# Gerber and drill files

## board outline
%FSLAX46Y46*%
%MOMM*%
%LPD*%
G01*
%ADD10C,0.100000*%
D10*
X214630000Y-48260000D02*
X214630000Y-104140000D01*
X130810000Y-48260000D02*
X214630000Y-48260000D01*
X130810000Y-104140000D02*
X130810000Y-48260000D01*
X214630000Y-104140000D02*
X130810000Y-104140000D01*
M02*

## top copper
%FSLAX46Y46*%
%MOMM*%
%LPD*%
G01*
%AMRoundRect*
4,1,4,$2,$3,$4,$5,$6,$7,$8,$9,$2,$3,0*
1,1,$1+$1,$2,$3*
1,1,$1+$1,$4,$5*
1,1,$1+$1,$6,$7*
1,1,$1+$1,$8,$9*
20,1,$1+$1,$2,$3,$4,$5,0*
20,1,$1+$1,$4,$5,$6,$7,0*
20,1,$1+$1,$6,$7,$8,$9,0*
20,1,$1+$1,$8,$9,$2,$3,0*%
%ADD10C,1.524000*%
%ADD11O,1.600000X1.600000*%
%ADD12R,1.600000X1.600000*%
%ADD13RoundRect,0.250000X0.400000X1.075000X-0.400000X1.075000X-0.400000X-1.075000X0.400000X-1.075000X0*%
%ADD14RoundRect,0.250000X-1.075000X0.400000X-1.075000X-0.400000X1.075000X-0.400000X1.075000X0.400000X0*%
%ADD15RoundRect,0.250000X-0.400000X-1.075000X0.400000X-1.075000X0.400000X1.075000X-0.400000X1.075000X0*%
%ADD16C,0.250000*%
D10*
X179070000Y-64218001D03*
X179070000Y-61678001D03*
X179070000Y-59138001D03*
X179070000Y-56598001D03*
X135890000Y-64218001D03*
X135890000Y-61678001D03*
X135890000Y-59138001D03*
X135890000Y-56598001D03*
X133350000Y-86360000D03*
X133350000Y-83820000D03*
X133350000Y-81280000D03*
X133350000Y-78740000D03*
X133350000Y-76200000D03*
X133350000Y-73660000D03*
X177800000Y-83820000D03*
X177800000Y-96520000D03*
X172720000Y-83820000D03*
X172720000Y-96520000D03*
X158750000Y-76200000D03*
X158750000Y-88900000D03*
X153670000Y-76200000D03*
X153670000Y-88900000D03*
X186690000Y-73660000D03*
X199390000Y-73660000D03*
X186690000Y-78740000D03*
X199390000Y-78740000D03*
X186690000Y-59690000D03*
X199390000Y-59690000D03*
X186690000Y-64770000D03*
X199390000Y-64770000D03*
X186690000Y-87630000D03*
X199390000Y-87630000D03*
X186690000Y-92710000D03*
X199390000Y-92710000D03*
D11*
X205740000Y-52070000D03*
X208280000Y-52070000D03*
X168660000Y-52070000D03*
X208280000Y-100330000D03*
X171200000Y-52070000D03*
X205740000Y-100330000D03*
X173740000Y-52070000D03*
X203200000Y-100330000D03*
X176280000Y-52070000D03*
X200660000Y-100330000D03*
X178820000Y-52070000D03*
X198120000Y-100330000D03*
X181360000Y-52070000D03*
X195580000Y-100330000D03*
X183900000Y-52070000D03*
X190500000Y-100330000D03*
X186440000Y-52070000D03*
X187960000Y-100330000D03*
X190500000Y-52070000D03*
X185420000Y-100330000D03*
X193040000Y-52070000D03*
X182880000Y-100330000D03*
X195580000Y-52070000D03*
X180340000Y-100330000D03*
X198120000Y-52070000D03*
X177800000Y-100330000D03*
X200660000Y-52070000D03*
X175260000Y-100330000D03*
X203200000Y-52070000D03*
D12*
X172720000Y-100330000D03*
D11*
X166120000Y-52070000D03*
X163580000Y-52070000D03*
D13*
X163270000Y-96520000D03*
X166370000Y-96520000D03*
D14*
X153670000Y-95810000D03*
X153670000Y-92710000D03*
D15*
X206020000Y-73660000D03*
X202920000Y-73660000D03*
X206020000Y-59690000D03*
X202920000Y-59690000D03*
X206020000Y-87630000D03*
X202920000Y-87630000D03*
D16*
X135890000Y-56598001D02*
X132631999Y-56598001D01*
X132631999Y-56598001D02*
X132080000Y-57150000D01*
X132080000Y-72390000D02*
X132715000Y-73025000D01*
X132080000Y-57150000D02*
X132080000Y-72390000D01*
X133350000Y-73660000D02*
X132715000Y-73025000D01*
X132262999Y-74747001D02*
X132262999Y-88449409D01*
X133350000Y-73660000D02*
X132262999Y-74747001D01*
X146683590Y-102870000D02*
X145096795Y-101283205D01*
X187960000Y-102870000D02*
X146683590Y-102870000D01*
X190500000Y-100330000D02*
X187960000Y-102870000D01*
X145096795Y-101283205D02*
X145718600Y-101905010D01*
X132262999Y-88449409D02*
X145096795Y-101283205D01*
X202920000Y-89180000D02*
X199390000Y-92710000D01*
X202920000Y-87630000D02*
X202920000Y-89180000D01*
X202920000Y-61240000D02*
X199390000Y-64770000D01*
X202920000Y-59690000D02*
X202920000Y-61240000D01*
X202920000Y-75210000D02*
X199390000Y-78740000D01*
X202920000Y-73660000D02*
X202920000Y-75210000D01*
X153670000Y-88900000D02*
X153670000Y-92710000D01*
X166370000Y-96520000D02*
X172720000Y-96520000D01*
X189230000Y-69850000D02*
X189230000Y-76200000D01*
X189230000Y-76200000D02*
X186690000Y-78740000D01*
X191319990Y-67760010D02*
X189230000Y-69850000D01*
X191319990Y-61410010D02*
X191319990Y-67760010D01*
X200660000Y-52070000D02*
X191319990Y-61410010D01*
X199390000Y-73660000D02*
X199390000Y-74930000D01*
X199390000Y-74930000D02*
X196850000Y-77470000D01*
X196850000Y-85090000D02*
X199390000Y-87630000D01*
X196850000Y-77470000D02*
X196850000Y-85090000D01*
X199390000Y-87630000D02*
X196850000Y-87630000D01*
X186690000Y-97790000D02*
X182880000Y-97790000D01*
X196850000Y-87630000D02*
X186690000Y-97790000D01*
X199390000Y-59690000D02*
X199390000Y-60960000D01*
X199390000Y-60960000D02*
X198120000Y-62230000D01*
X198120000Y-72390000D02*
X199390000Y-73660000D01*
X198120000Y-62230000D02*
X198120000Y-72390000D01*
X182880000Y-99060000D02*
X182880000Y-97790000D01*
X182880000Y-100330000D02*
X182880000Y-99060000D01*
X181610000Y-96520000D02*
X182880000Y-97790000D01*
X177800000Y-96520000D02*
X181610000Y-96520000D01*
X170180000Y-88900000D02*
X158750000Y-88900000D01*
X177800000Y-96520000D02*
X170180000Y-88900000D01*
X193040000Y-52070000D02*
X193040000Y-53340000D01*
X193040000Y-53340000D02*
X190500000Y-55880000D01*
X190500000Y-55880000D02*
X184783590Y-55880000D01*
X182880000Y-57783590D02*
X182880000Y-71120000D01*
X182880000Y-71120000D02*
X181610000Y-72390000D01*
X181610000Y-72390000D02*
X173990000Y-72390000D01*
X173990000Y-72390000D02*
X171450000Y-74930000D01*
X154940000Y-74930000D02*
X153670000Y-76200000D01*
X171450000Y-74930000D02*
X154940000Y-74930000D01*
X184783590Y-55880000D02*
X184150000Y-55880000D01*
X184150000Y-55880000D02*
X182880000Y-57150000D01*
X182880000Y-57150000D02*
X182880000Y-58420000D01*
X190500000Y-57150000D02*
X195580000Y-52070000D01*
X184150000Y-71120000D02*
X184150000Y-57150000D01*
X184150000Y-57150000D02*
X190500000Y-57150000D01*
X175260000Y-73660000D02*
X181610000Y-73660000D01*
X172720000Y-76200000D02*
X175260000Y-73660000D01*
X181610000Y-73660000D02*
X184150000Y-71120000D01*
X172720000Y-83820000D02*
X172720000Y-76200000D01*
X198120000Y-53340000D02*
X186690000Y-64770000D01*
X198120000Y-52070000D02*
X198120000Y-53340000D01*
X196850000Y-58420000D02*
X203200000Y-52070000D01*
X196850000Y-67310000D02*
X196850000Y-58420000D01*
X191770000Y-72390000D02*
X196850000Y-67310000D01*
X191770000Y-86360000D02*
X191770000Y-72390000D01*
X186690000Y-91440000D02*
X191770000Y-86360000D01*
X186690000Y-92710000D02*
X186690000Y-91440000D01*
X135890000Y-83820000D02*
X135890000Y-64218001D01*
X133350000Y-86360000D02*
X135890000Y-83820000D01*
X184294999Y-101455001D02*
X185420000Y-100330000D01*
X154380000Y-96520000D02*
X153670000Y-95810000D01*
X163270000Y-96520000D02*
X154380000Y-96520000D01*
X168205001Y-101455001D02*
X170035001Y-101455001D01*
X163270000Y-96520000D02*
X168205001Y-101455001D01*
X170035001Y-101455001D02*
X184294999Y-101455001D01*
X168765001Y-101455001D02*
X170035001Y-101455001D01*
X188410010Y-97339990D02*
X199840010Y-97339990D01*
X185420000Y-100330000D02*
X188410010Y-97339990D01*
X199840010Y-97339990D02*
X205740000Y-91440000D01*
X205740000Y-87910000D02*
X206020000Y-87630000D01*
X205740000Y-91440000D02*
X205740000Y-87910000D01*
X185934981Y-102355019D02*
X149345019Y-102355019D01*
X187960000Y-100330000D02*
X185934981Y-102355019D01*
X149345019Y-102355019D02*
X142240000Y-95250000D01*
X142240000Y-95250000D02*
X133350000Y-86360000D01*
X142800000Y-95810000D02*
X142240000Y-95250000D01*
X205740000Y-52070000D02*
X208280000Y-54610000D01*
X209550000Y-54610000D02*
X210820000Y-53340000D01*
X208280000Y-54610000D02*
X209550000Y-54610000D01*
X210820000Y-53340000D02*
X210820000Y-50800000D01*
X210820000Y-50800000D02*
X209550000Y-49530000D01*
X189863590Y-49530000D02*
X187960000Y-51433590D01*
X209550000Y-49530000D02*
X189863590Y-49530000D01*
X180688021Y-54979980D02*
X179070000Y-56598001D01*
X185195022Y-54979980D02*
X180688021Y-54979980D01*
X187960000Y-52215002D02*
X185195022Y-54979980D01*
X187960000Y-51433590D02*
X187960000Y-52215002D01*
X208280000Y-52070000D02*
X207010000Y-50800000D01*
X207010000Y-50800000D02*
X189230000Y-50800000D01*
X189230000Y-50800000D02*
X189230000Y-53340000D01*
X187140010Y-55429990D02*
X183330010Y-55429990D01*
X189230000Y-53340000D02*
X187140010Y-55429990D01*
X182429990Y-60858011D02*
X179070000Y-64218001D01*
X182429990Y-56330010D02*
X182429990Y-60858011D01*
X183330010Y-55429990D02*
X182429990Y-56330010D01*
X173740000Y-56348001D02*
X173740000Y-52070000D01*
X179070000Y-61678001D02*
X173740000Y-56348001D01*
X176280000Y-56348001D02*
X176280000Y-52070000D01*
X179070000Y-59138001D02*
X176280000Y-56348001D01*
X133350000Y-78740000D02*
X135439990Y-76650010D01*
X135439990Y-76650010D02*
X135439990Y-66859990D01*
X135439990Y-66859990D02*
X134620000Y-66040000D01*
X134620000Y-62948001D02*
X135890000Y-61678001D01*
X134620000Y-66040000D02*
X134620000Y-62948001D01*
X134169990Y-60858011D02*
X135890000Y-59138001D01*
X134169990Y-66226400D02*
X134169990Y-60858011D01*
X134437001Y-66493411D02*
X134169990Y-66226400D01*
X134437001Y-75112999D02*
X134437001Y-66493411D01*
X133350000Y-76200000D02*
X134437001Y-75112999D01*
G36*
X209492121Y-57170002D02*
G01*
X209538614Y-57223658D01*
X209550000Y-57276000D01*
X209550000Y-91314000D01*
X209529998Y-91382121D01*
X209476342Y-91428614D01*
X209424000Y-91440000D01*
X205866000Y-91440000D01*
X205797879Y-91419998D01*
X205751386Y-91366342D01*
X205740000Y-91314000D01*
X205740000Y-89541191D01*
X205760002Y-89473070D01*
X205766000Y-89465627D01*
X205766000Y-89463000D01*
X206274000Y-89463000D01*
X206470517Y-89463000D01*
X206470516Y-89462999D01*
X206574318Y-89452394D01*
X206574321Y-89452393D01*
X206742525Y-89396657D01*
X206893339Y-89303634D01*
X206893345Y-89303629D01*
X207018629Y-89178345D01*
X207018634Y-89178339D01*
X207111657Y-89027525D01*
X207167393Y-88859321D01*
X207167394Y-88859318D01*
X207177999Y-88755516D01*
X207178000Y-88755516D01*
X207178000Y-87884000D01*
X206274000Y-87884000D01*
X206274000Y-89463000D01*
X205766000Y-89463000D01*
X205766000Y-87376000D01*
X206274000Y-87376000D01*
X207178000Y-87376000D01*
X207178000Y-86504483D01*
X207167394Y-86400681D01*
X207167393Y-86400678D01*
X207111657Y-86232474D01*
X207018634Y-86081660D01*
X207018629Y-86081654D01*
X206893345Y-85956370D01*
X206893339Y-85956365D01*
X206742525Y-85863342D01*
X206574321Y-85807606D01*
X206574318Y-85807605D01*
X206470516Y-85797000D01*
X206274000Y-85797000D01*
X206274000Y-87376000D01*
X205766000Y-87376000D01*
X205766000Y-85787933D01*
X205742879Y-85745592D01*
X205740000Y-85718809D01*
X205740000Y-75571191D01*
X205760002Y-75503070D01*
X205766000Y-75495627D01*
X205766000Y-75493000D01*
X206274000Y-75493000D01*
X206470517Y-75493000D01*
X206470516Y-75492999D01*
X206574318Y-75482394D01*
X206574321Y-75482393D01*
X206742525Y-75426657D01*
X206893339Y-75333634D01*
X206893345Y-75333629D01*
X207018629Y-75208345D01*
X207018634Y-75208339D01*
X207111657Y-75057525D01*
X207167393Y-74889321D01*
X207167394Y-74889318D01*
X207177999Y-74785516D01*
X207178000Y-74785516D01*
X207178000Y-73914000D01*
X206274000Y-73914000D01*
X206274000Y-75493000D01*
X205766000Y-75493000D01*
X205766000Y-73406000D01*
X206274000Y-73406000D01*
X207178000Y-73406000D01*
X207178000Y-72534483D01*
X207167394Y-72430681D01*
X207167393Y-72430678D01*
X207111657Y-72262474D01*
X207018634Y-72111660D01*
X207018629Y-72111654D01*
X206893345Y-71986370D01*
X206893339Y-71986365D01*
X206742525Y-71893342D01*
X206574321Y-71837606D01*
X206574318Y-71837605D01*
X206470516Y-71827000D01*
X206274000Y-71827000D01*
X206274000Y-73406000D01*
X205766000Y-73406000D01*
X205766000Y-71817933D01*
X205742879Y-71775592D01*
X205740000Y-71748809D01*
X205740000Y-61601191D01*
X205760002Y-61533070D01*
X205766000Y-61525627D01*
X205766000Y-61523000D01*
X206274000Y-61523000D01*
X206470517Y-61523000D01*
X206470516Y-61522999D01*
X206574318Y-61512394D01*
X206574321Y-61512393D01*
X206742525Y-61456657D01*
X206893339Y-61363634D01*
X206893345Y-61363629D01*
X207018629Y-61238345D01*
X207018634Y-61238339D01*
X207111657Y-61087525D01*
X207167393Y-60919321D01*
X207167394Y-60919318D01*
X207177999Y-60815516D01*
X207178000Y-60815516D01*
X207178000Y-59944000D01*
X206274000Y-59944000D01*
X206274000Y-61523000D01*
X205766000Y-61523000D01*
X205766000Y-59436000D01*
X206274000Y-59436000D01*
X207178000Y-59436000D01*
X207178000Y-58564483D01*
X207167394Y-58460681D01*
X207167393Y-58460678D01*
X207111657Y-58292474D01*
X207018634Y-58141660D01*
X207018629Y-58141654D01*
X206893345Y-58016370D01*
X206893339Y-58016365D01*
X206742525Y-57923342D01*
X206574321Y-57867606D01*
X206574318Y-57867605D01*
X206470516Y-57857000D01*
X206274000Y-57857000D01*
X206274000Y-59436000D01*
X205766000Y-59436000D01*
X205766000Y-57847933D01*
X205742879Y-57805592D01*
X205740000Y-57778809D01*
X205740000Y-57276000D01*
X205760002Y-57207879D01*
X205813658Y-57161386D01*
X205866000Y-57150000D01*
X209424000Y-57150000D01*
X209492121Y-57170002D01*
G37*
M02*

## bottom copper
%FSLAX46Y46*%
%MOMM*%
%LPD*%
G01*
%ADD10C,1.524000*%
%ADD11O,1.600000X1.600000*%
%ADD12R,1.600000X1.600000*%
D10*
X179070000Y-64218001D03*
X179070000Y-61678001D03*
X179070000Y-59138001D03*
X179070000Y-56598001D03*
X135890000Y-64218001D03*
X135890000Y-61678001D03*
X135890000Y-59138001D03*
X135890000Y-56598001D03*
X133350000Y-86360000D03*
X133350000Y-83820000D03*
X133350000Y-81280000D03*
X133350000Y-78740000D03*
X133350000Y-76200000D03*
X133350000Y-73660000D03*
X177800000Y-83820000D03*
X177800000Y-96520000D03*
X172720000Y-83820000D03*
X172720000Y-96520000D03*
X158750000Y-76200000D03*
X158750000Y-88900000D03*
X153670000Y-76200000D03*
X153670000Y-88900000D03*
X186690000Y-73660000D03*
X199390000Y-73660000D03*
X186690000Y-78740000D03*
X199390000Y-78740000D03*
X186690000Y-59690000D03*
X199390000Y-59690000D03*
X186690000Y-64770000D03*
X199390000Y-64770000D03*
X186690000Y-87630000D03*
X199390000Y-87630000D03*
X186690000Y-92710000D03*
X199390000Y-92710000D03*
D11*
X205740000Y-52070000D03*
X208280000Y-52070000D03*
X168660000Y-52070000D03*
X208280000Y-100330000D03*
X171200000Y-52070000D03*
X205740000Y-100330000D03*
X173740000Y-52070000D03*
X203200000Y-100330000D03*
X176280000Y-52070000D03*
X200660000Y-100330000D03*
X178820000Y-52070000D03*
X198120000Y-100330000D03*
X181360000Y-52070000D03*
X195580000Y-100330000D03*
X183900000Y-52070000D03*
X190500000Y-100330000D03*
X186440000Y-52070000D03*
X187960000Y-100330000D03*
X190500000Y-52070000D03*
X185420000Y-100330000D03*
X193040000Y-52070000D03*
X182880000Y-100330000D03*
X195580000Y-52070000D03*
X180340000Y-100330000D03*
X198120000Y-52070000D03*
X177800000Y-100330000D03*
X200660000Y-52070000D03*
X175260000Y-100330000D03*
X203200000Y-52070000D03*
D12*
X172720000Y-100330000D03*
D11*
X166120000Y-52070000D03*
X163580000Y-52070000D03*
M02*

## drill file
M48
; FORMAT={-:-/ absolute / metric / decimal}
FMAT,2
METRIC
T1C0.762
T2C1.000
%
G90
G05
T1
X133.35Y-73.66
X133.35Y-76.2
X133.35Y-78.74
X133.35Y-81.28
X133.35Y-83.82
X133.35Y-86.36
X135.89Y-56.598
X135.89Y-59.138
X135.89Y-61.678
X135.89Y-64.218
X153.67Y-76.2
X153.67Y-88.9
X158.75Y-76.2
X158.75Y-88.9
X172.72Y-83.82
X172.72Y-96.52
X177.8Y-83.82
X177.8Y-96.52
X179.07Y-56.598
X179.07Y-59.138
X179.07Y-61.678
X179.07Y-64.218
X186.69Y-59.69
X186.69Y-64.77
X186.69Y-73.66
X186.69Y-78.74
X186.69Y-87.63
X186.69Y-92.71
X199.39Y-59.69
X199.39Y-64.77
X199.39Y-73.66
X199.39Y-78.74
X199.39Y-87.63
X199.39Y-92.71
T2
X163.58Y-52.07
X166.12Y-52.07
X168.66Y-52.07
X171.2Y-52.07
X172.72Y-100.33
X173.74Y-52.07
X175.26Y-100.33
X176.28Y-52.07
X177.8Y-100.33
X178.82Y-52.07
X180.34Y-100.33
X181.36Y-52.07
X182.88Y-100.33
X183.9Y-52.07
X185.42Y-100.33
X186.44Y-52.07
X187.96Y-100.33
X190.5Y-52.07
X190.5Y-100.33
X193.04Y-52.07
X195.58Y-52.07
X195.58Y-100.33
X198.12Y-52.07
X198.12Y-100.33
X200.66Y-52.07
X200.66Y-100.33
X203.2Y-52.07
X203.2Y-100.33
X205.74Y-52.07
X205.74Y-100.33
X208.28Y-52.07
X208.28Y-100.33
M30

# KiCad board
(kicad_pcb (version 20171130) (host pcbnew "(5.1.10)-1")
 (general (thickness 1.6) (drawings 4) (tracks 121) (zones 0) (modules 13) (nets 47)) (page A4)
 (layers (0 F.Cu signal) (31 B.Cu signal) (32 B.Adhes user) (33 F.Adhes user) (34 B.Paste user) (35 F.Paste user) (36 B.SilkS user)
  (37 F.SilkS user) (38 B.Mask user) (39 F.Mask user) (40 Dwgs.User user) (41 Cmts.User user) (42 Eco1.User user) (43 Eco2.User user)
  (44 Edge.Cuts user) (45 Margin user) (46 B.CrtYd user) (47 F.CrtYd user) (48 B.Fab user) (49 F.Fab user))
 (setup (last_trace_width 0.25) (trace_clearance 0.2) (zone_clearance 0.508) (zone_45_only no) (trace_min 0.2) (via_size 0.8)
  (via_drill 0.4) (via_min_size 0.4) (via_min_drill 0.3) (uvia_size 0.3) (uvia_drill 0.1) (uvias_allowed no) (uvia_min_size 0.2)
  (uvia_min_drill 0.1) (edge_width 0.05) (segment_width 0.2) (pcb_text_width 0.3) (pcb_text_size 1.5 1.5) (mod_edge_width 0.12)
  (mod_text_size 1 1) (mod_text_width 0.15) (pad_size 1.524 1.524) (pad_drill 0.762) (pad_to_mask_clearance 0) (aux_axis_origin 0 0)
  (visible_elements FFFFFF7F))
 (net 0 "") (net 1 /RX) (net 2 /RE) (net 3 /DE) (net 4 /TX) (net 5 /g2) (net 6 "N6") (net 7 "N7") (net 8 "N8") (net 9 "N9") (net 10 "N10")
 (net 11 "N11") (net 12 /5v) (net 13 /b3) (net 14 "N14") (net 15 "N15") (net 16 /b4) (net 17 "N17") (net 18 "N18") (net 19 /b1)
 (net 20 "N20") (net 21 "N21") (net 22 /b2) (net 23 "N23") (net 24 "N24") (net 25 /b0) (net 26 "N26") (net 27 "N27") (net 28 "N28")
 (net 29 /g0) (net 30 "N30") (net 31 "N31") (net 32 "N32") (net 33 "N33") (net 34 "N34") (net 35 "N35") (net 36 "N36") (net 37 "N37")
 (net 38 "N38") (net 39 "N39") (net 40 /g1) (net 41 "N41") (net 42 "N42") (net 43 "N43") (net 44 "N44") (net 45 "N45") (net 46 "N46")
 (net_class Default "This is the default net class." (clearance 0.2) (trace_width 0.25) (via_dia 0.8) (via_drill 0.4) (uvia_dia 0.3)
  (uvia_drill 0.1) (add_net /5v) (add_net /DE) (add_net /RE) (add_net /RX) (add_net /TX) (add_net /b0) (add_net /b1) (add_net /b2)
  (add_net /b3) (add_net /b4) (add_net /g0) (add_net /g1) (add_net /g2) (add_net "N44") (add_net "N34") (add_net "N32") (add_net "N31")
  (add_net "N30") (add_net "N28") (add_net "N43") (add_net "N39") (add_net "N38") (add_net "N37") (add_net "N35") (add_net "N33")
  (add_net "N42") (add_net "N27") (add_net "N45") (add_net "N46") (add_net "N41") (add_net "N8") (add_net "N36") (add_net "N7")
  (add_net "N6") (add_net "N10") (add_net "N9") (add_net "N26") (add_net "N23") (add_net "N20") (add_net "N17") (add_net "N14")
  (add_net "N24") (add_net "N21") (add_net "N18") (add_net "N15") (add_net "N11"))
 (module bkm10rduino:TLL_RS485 (layer F.Cu) (at 157.48 61.678001)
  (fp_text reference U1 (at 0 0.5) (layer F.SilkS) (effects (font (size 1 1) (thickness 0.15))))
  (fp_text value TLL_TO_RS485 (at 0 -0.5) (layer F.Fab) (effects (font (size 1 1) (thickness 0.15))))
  (pad 8 thru_hole circle (at 21.59 2.54) (size 1.524 1.524) (drill 0.762) (layers *.Cu *.Mask) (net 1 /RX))
  (pad 7 thru_hole circle (at 21.59 0) (size 1.524 1.524) (drill 0.762) (layers *.Cu *.Mask) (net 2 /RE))
  (pad 6 thru_hole circle (at 21.59 -2.54) (size 1.524 1.524) (drill 0.762) (layers *.Cu *.Mask) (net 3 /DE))
  (pad 5 thru_hole circle (at 21.59 -5.08) (size 1.524 1.524) (drill 0.762) (layers *.Cu *.Mask) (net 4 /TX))
  (pad 4 thru_hole circle (at -21.59 2.54) (size 1.524 1.524) (drill 0.762) (layers *.Cu *.Mask) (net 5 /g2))
  (pad 3 thru_hole circle (at -21.59 0) (size 1.524 1.524) (drill 0.762) (layers *.Cu *.Mask) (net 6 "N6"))
  (pad 2 thru_hole circle (at -21.59 -2.54) (size 1.524 1.524) (drill 0.762) (layers *.Cu *.Mask) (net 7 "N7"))
  (pad 1 thru_hole circle (at -21.59 -5.08) (size 1.524 1.524) (drill 0.762) (layers *.Cu *.Mask) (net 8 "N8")))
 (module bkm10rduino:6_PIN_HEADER (layer F.Cu) (at 129.54 78.74 270)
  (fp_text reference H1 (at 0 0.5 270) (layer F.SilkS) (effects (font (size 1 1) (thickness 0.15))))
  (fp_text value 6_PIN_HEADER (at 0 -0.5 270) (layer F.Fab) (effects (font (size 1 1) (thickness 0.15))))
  (pad 6 thru_hole circle (at 7.62 -3.81 270) (size 1.524 1.524) (drill 0.762) (layers *.Cu *.Mask) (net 5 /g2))
  (pad 5 thru_hole circle (at 5.08 -3.81 270) (size 1.524 1.524) (drill 0.762) (layers *.Cu *.Mask) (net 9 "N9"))
  (pad 4 thru_hole circle (at 2.54 -3.81 270) (size 1.524 1.524) (drill 0.762) (layers *.Cu *.Mask) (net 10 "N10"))
  (pad 3 thru_hole circle (at 0 -3.81 270) (size 1.524 1.524) (drill 0.762) (layers *.Cu *.Mask) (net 6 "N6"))
  (pad 2 thru_hole circle (at -2.54 -3.81 270) (size 1.524 1.524) (drill 0.762) (layers *.Cu *.Mask) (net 7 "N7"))
  (pad 1 thru_hole circle (at -5.08 -3.81 270) (size 1.524 1.524) (drill 0.762) (layers *.Cu *.Mask) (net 8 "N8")))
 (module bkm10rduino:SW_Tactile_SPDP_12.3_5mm (layer F.Cu) (at 175.26 90.17)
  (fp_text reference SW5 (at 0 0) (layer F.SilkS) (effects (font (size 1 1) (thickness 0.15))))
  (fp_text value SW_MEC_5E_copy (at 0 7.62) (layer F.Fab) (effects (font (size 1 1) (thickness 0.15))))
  (pad 4 thru_hole circle (at 2.54 -6.35) (size 1.524 1.524) (drill 0.762) (layers *.Cu *.Mask) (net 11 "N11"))
  (pad 3 thru_hole circle (at 2.54 6.35) (size 1.524 1.524) (drill 0.762) (layers *.Cu *.Mask) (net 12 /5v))
  (pad 2 thru_hole circle (at -2.54 -6.35) (size 1.524 1.524) (drill 0.762) (layers *.Cu *.Mask) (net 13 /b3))
  (pad 1 thru_hole circle (at -2.54 6.35) (size 1.524 1.524) (drill 0.762) (layers *.Cu *.Mask) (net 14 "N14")))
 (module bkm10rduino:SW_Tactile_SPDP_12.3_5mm (layer F.Cu) (at 156.21 82.55)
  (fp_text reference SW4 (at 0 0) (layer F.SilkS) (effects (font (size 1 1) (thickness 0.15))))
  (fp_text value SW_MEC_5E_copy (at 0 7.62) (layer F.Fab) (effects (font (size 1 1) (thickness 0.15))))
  (pad 4 thru_hole circle (at 2.54 -6.35) (size 1.524 1.524) (drill 0.762) (layers *.Cu *.Mask) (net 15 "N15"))
  (pad 3 thru_hole circle (at 2.54 6.35) (size 1.524 1.524) (drill 0.762) (layers *.Cu *.Mask) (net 12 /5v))
  (pad 2 thru_hole circle (at -2.54 -6.35) (size 1.524 1.524) (drill 0.762) (layers *.Cu *.Mask) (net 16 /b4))
  (pad 1 thru_hole circle (at -2.54 6.35) (size 1.524 1.524) (drill 0.762) (layers *.Cu *.Mask) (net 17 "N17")))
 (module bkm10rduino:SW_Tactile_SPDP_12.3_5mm (layer F.Cu) (at 193.04 76.2 90)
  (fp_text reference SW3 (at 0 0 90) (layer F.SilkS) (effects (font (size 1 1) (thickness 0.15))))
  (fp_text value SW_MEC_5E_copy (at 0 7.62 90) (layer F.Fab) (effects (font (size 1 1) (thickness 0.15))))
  (pad 4 thru_hole circle (at 2.54 -6.35 90) (size 1.524 1.524) (drill 0.762) (layers *.Cu *.Mask) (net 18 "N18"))
  (pad 3 thru_hole circle (at 2.54 6.35 90) (size 1.524 1.524) (drill 0.762) (layers *.Cu *.Mask) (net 12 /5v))
  (pad 2 thru_hole circle (at -2.54 -6.35 90) (size 1.524 1.524) (drill 0.762) (layers *.Cu *.Mask) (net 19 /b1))
  (pad 1 thru_hole circle (at -2.54 6.35 90) (size 1.524 1.524) (drill 0.762) (layers *.Cu *.Mask) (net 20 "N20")))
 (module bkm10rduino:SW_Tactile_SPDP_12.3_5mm (layer F.Cu) (at 193.04 62.23 90)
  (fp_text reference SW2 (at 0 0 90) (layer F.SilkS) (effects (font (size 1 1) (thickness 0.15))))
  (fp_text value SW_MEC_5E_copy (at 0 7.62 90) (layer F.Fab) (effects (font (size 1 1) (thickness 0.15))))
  (pad 4 thru_hole circle (at 2.54 -6.35 90) (size 1.524 1.524) (drill 0.762) (layers *.Cu *.Mask) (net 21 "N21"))
  (pad 3 thru_hole circle (at 2.54 6.35 90) (size 1.524 1.524) (drill 0.762) (layers *.Cu *.Mask) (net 12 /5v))
  (pad 2 thru_hole circle (at -2.54 -6.35 90) (size 1.524 1.524) (drill 0.762) (layers *.Cu *.Mask) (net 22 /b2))
  (pad 1 thru_hole circle (at -2.54 6.35 90) (size 1.524 1.524) (drill 0.762) (layers *.Cu *.Mask) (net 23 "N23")))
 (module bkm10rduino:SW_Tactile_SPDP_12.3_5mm (layer F.Cu) (at 193.04 90.17 90)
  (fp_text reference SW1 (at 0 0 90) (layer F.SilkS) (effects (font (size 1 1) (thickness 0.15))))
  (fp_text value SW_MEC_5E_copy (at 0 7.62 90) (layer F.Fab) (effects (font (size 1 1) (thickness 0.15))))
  (pad 4 thru_hole circle (at 2.54 -6.35 90) (size 1.524 1.524) (drill 0.762) (layers *.Cu *.Mask) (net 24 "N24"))
  (pad 3 thru_hole circle (at 2.54 6.35 90) (size 1.524 1.524) (drill 0.762) (layers *.Cu *.Mask) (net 12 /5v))
  (pad 2 thru_hole circle (at -2.54 -6.35 90) (size 1.524 1.524) (drill 0.762) (layers *.Cu *.Mask) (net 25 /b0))
  (pad 1 thru_hole circle (at -2.54 6.35 90) (size 1.524 1.524) (drill 0.762) (layers *.Cu *.Mask) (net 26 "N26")))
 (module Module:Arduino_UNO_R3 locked (layer B.Cu) (at 172.72 100.33)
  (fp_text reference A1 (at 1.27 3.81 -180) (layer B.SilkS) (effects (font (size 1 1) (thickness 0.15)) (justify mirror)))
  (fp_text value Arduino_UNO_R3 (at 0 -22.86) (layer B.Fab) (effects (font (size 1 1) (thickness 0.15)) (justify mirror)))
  (pad 16 thru_hole oval (at 33.02 -48.26 270) (size 1.6 1.6) (drill 1) (layers *.Cu *.Mask) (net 4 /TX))
  (pad 15 thru_hole oval (at 35.56 -48.26 270) (size 1.6 1.6) (drill 1) (layers *.Cu *.Mask) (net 1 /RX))
  (pad 30 thru_hole oval (at -4.06 -48.26 270) (size 1.6 1.6) (drill 1) (layers *.Cu *.Mask) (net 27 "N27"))
  (pad 14 thru_hole oval (at 35.56 0 270) (size 1.6 1.6) (drill 1) (layers *.Cu *.Mask) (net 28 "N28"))
  (pad 29 thru_hole oval (at -1.52 -48.26 270) (size 1.6 1.6) (drill 1) (layers *.Cu *.Mask) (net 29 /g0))
  (pad 13 thru_hole oval (at 33.02 0 270) (size 1.6 1.6) (drill 1) (layers *.Cu *.Mask) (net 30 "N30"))
  (pad 28 thru_hole oval (at 1.02 -48.26 270) (size 1.6 1.6) (drill 1) (layers *.Cu *.Mask) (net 2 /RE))
  (pad 12 thru_hole oval (at 30.48 0 270) (size 1.6 1.6) (drill 1) (layers *.Cu *.Mask) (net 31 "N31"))
  (pad 27 thru_hole oval (at 3.56 -48.26 270) (size 1.6 1.6) (drill 1) (layers *.Cu *.Mask) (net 3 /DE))
  (pad 11 thru_hole oval (at 27.94 0 270) (size 1.6 1.6) (drill 1) (layers *.Cu *.Mask) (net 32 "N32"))
  (pad 26 thru_hole oval (at 6.1 -48.26 270) (size 1.6 1.6) (drill 1) (layers *.Cu *.Mask) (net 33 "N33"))
  (pad 10 thru_hole oval (at 25.4 0 270) (size 1.6 1.6) (drill 1) (layers *.Cu *.Mask) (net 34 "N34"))
  (pad 25 thru_hole oval (at 8.64 -48.26 270) (size 1.6 1.6) (drill 1) (layers *.Cu *.Mask) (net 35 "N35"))
  (pad 9 thru_hole oval (at 22.86 0 270) (size 1.6 1.6) (drill 1) (layers *.Cu *.Mask) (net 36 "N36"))
  (pad 24 thru_hole oval (at 11.18 -48.26 270) (size 1.6 1.6) (drill 1) (layers *.Cu *.Mask) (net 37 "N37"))
  (pad 8 thru_hole oval (at 17.78 0 270) (size 1.6 1.6) (drill 1) (layers *.Cu *.Mask) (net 8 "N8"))
  (pad 23 thru_hole oval (at 13.72 -48.26 270) (size 1.6 1.6) (drill 1) (layers *.Cu *.Mask) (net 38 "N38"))
  (pad 7 thru_hole oval (at 15.24 0 270) (size 1.6 1.6) (drill 1) (layers *.Cu *.Mask) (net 5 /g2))
  (pad 22 thru_hole oval (at 17.78 -48.26 270) (size 1.6 1.6) (drill 1) (layers *.Cu *.Mask) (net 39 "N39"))
  (pad 6 thru_hole oval (at 12.7 0 270) (size 1.6 1.6) (drill 1) (layers *.Cu *.Mask) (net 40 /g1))
  (pad 21 thru_hole oval (at 20.32 -48.26 270) (size 1.6 1.6) (drill 1) (layers *.Cu *.Mask) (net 16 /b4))
  (pad 5 thru_hole oval (at 10.16 0 270) (size 1.6 1.6) (drill 1) (layers *.Cu *.Mask) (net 12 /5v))
  (pad 20 thru_hole oval (at 22.86 -48.26 270) (size 1.6 1.6) (drill 1) (layers *.Cu *.Mask) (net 13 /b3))
  (pad 4 thru_hole oval (at 7.62 0 270) (size 1.6 1.6) (drill 1) (layers *.Cu *.Mask) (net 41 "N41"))
  (pad 19 thru_hole oval (at 25.4 -48.26 270) (size 1.6 1.6) (drill 1) (layers *.Cu *.Mask) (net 22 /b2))
  (pad 3 thru_hole oval (at 5.08 0 270) (size 1.6 1.6) (drill 1) (layers *.Cu *.Mask) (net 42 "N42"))
  (pad 18 thru_hole oval (at 27.94 -48.26 270) (size 1.6 1.6) (drill 1) (layers *.Cu *.Mask) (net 19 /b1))
  (pad 2 thru_hole oval (at 2.54 0 270) (size 1.6 1.6) (drill 1) (layers *.Cu *.Mask) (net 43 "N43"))
  (pad 17 thru_hole oval (at 30.48 -48.26 270) (size 1.6 1.6) (drill 1) (layers *.Cu *.Mask) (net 25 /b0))
  (pad 1 thru_hole rect (at 0 0 270) (size 1.6 1.6) (drill 1) (layers *.Cu *.Mask) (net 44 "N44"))
  (pad 31 thru_hole oval (at -6.6 -48.26 270) (size 1.6 1.6) (drill 1) (layers *.Cu *.Mask) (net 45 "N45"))
  (pad 32 thru_hole oval (at -9.14 -48.26 270) (size 1.6 1.6) (drill 1) (layers *.Cu *.Mask) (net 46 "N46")))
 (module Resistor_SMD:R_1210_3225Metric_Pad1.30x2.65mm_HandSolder (layer F.Cu) (at 164.82 96.52 180)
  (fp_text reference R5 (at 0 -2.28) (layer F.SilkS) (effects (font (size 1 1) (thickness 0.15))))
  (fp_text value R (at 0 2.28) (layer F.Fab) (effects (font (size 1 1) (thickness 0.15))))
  (pad 2 smd roundrect (at 1.55 0 180) (size 1.3 2.65) (layers F.Cu F.Paste F.Mask) (roundrect_rratio 0.192308) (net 40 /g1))
  (pad 1 smd roundrect (at -1.55 0 180) (size 1.3 2.65) (layers F.Cu F.Paste F.Mask) (roundrect_rratio 0.192308) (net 14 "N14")))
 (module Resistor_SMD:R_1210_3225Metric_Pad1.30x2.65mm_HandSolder (layer F.Cu) (at 153.67 94.26 270)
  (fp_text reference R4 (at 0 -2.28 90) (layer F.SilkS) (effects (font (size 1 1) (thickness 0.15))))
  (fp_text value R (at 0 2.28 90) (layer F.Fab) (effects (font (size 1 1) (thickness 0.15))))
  (pad 2 smd roundrect (at 1.55 0 270) (size 1.3 2.65) (layers F.Cu F.Paste F.Mask) (roundrect_rratio 0.192308) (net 40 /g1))
  (pad 1 smd roundrect (at -1.55 0 270) (size 1.3 2.65) (layers F.Cu F.Paste F.Mask) (roundrect_rratio 0.192308) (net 17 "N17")))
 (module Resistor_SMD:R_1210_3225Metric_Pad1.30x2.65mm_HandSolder (layer F.Cu) (at 204.47 73.66)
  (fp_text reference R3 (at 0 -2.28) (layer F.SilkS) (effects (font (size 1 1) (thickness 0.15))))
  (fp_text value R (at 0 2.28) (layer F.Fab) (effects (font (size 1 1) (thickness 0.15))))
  (pad 2 smd roundrect (at 1.55 0) (size 1.3 2.65) (layers F.Cu F.Paste F.Mask) (roundrect_rratio 0.192308) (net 40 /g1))
  (pad 1 smd roundrect (at -1.55 0) (size 1.3 2.65) (layers F.Cu F.Paste F.Mask) (roundrect_rratio 0.192308) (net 20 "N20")))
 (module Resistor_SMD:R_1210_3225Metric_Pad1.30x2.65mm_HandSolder (layer F.Cu) (at 204.47 59.69)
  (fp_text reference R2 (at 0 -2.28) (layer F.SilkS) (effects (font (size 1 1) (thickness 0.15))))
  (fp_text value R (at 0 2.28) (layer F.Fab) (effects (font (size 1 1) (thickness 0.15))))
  (pad 2 smd roundrect (at 1.55 0) (size 1.3 2.65) (layers F.Cu F.Paste F.Mask) (roundrect_rratio 0.192308) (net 40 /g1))
  (pad 1 smd roundrect (at -1.55 0) (size 1.3 2.65) (layers F.Cu F.Paste F.Mask) (roundrect_rratio 0.192308) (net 23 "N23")))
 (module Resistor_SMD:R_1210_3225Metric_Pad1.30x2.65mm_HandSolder (layer F.Cu) (at 204.47 87.63)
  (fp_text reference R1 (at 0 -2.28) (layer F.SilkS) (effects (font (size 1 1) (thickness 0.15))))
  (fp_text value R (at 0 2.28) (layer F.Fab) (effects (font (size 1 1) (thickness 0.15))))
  (pad 2 smd roundrect (at 1.55 0) (size 1.3 2.65) (layers F.Cu F.Paste F.Mask) (roundrect_rratio 0.192308) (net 40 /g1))
  (pad 1 smd roundrect (at -1.55 0) (size 1.3 2.65) (layers F.Cu F.Paste F.Mask) (roundrect_rratio 0.192308) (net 26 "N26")))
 (gr_line (start 214.63 48.26) (end 214.63 104.14) (layer Edge.Cuts) (width 0.1))
 (gr_line (start 130.81 48.26) (end 214.63 48.26) (layer Edge.Cuts) (width 0.1))
 (gr_line (start 130.81 104.14) (end 130.81 48.26) (layer Edge.Cuts) (width 0.1))
 (gr_line (start 214.63 104.14) (end 130.81 104.14) (layer Edge.Cuts) (width 0.1))
 (segment (start 135.89 56.598001) (end 132.631999 56.598001) (width 0.25) (layer F.Cu) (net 8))
 (segment (start 132.631999 56.598001) (end 132.08 57.15) (width 0.25) (layer F.Cu) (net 8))
 (segment (start 132.08 72.39) (end 132.715 73.025) (width 0.25) (layer F.Cu) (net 8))
 (segment (start 132.08 57.15) (end 132.08 72.39) (width 0.25) (layer F.Cu) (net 8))
 (segment (start 133.35 73.66) (end 132.715 73.025) (width 0.25) (layer F.Cu) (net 8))
 (segment (start 132.262999 74.747001) (end 132.262999 88.449409) (width 0.25) (layer F.Cu) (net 8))
 (segment (start 133.35 73.66) (end 132.262999 74.747001) (width 0.25) (layer F.Cu) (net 8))
 (segment (start 146.68359 102.87) (end 145.096795 101.283205) (width 0.25) (layer F.Cu) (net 8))
 (segment (start 187.96 102.87) (end 146.68359 102.87) (width 0.25) (layer F.Cu) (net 8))
 (segment (start 190.5 100.33) (end 187.96 102.87) (width 0.25) (layer F.Cu) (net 8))
 (segment (start 145.096795 101.283205) (end 145.7186 101.90501) (width 0.25) (layer F.Cu) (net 8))
 (segment (start 132.262999 88.449409) (end 145.096795 101.283205) (width 0.25) (layer F.Cu) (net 8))
 (segment (start 202.92 89.18) (end 199.39 92.71) (width 0.25) (layer F.Cu) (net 26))
 (segment (start 202.92 87.63) (end 202.92 89.18) (width 0.25) (layer F.Cu) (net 26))
 (segment (start 202.92 61.24) (end 199.39 64.77) (width 0.25) (layer F.Cu) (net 23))
 (segment (start 202.92 59.69) (end 202.92 61.24) (width 0.25) (layer F.Cu) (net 23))
 (segment (start 202.92 75.21) (end 199.39 78.74) (width 0.25) (layer F.Cu) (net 20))
 (segment (start 202.92 73.66) (end 202.92 75.21) (width 0.25) (layer F.Cu) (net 20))
 (segment (start 153.67 88.9) (end 153.67 92.71) (width 0.25) (layer F.Cu) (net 17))
 (segment (start 166.37 96.52) (end 172.72 96.52) (width 0.25) (layer F.Cu) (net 14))
 (segment (start 189.23 69.85) (end 189.23 76.2) (width 0.25) (layer F.Cu) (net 19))
 (segment (start 189.23 76.2) (end 186.69 78.74) (width 0.25) (layer F.Cu) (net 19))
 (segment (start 191.31999 67.76001) (end 189.23 69.85) (width 0.25) (layer F.Cu) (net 19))
 (segment (start 191.31999 61.41001) (end 191.31999 67.76001) (width 0.25) (layer F.Cu) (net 19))
 (segment (start 200.66 52.07) (end 191.31999 61.41001) (width 0.25) (layer F.Cu) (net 19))
 (segment (start 199.39 73.66) (end 199.39 74.93) (width 0.25) (layer F.Cu) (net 12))
 (segment (start 199.39 74.93) (end 196.85 77.47) (width 0.25) (layer F.Cu) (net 12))
 (segment (start 196.85 85.09) (end 199.39 87.63) (width 0.25) (layer F.Cu) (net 12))
 (segment (start 196.85 77.47) (end 196.85 85.09) (width 0.25) (layer F.Cu) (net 12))
 (segment (start 199.39 87.63) (end 196.85 87.63) (width 0.25) (layer F.Cu) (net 12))
 (segment (start 186.69 97.79) (end 182.88 97.79) (width 0.25) (layer F.Cu) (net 12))
 (segment (start 196.85 87.63) (end 186.69 97.79) (width 0.25) (layer F.Cu) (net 12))
 (segment (start 199.39 59.69) (end 199.39 60.96) (width 0.25) (layer F.Cu) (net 12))
 (segment (start 199.39 60.96) (end 198.12 62.23) (width 0.25) (layer F.Cu) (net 12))
 (segment (start 198.12 72.39) (end 199.39 73.66) (width 0.25) (layer F.Cu) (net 12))
 (segment (start 198.12 62.23) (end 198.12 72.39) (width 0.25) (layer F.Cu) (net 12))
 (segment (start 182.88 99.06) (end 182.88 97.79) (width 0.25) (layer F.Cu) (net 12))
 (segment (start 182.88 100.33) (end 182.88 99.06) (width 0.25) (layer F.Cu) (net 12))
 (segment (start 181.61 96.52) (end 182.88 97.79) (width 0.25) (layer F.Cu) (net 12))
 (segment (start 177.8 96.52) (end 181.61 96.52) (width 0.25) (layer F.Cu) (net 12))
 (segment (start 170.18 88.9) (end 158.75 88.9) (width 0.25) (layer F.Cu) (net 12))
 (segment (start 177.8 96.52) (end 170.18 88.9) (width 0.25) (layer F.Cu) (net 12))
 (segment (start 193.04 52.07) (end 193.04 53.34) (width 0.25) (layer F.Cu) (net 16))
 (segment (start 193.04 53.34) (end 190.5 55.88) (width 0.25) (layer F.Cu) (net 16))
 (segment (start 190.5 55.88) (end 184.78359 55.88) (width 0.25) (layer F.Cu) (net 16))
 (segment (start 182.88 57.78359) (end 182.88 71.12) (width 0.25) (layer F.Cu) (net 16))
 (segment (start 182.88 71.12) (end 181.61 72.39) (width 0.25) (layer F.Cu) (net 16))
 (segment (start 181.61 72.39) (end 173.99 72.39) (width 0.25) (layer F.Cu) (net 16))
 (segment (start 173.99 72.39) (end 171.45 74.93) (width 0.25) (layer F.Cu) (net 16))
 (segment (start 154.94 74.93) (end 153.67 76.2) (width 0.25) (layer F.Cu) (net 16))
 (segment (start 171.45 74.93) (end 154.94 74.93) (width 0.25) (layer F.Cu) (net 16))
 (segment (start 184.78359 55.88) (end 184.15 55.88) (width 0.25) (layer F.Cu) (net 16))
 (segment (start 184.15 55.88) (end 182.88 57.15) (width 0.25) (layer F.Cu) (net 16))
 (segment (start 182.88 57.15) (end 182.88 58.42) (width 0.25) (layer F.Cu) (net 16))
 (segment (start 190.5 57.15) (end 195.58 52.07) (width 0.25) (layer F.Cu) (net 13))
 (segment (start 184.15 71.12) (end 184.15 57.15) (width 0.25) (layer F.Cu) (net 13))
 (segment (start 184.15 57.15) (end 190.5 57.15) (width 0.25) (layer F.Cu) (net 13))
 (segment (start 175.26 73.66) (end 181.61 73.66) (width 0.25) (layer F.Cu) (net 13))
 (segment (start 172.72 76.2) (end 175.26 73.66) (width 0.25) (layer F.Cu) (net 13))
 (segment (start 181.61 73.66) (end 184.15 71.12) (width 0.25) (layer F.Cu) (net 13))
 (segment (start 172.72 83.82) (end 172.72 76.2) (width 0.25) (layer F.Cu) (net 13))
 (segment (start 198.12 53.34) (end 186.69 64.77) (width 0.25) (layer F.Cu) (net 22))
 (segment (start 198.12 52.07) (end 198.12 53.34) (width 0.25) (layer F.Cu) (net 22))
 (segment (start 196.85 58.42) (end 203.2 52.07) (width 0.25) (layer F.Cu) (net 25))
 (segment (start 196.85 67.31) (end 196.85 58.42) (width 0.25) (layer F.Cu) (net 25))
 (segment (start 191.77 72.39) (end 196.85 67.31) (width 0.25) (layer F.Cu) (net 25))
 (segment (start 191.77 86.36) (end 191.77 72.39) (width 0.25) (layer F.Cu) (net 25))
 (segment (start 186.69 91.44) (end 191.77 86.36) (width 0.25) (layer F.Cu) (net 25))
 (segment (start 186.69 92.71) (end 186.69 91.44) (width 0.25) (layer F.Cu) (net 25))
 (segment (start 135.89 83.82) (end 135.89 64.218001) (width 0.25) (layer F.Cu) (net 5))
 (segment (start 133.35 86.36) (end 135.89 83.82) (width 0.25) (layer F.Cu) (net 5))
 (segment (start 184.294999 101.455001) (end 185.42 100.33) (width 0.25) (layer F.Cu) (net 40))
 (segment (start 154.38 96.52) (end 153.67 95.81) (width 0.25) (layer F.Cu) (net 40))
 (segment (start 163.27 96.52) (end 154.38 96.52) (width 0.25) (layer F.Cu) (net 40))
 (segment (start 168.205001 101.455001) (end 170.035001 101.455001) (width 0.25) (layer F.Cu) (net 40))
 (segment (start 163.27 96.52) (end 168.205001 101.455001) (width 0.25) (layer F.Cu) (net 40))
 (segment (start 170.035001 101.455001) (end 184.294999 101.455001) (width 0.25) (layer F.Cu) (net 40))
 (segment (start 168.765001 101.455001) (end 170.035001 101.455001) (width 0.25) (layer F.Cu) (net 40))
 (segment (start 188.41001 97.33999) (end 199.84001 97.33999) (width 0.25) (layer F.Cu) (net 40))
 (segment (start 185.42 100.33) (end 188.41001 97.33999) (width 0.25) (layer F.Cu) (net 40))
 (segment (start 199.84001 97.33999) (end 205.74 91.44) (width 0.25) (layer F.Cu) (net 40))
 (segment (start 205.74 87.91) (end 206.02 87.63) (width 0.25) (layer F.Cu) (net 40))
 (segment (start 205.74 91.44) (end 205.74 87.91) (width 0.25) (layer F.Cu) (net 40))
 (segment (start 185.934981 102.355019) (end 149.345019 102.355019) (width 0.25) (layer F.Cu) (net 5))
 (segment (start 187.96 100.33) (end 185.934981 102.355019) (width 0.25) (layer F.Cu) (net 5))
 (segment (start 149.345019 102.355019) (end 142.24 95.25) (width 0.25) (layer F.Cu) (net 5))
 (segment (start 142.24 95.25) (end 133.35 86.36) (width 0.25) (layer F.Cu) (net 5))
 (segment (start 142.8 95.81) (end 142.24 95.25) (width 0.25) (layer F.Cu) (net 5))
 (segment (start 205.74 52.07) (end 208.28 54.61) (width 0.25) (layer F.Cu) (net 4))
 (segment (start 209.55 54.61) (end 210.82 53.34) (width 0.25) (layer F.Cu) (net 4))
 (segment (start 208.28 54.61) (end 209.55 54.61) (width 0.25) (layer F.Cu) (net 4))
 (segment (start 210.82 53.34) (end 210.82 50.8) (width 0.25) (layer F.Cu) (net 4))
 (segment (start 210.82 50.8) (end 209.55 49.53) (width 0.25) (layer F.Cu) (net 4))
 (segment (start 189.86359 49.53) (end 187.96 51.43359) (width 0.25) (layer F.Cu) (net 4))
 (segment (start 209.55 49.53) (end 189.86359 49.53) (width 0.25) (layer F.Cu) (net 4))
 (segment (start 180.688021 54.97998) (end 179.07 56.598001) (width 0.25) (layer F.Cu) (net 4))
 (segment (start 185.195022 54.97998) (end 180.688021 54.97998) (width 0.25) (layer F.Cu) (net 4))
 (segment (start 187.96 52.215002) (end 185.195022 54.97998) (width 0.25) (layer F.Cu) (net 4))
 (segment (start 187.96 51.43359) (end 187.96 52.215002) (width 0.25) (layer F.Cu) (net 4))
 (segment (start 208.28 52.07) (end 207.01 50.8) (width 0.25) (layer F.Cu) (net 1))
 (segment (start 207.01 50.8) (end 189.23 50.8) (width 0.25) (layer F.Cu) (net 1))
 (segment (start 189.23 50.8) (end 189.23 53.34) (width 0.25) (layer F.Cu) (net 1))
 (segment (start 187.14001 55.42999) (end 183.33001 55.42999) (width 0.25) (layer F.Cu) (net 1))
 (segment (start 189.23 53.34) (end 187.14001 55.42999) (width 0.25) (layer F.Cu) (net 1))
 (segment (start 182.42999 60.858011) (end 179.07 64.218001) (width 0.25) (layer F.Cu) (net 1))
 (segment (start 182.42999 56.33001) (end 182.42999 60.858011) (width 0.25) (layer F.Cu) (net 1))
 (segment (start 183.33001 55.42999) (end 182.42999 56.33001) (width 0.25) (layer F.Cu) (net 1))
 (segment (start 173.74 56.348001) (end 173.74 52.07) (width 0.25) (layer F.Cu) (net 2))
 (segment (start 179.07 61.678001) (end 173.74 56.348001) (width 0.25) (layer F.Cu) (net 2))
 (segment (start 176.28 56.348001) (end 176.28 52.07) (width 0.25) (layer F.Cu) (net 3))
 (segment (start 179.07 59.138001) (end 176.28 56.348001) (width 0.25) (layer F.Cu) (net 3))
 (segment (start 133.35 78.74) (end 135.43999 76.65001) (width 0.25) (layer F.Cu) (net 6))
 (segment (start 135.43999 76.65001) (end 135.43999 66.85999) (width 0.25) (layer F.Cu) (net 6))
 (segment (start 135.43999 66.85999) (end 134.62 66.04) (width 0.25) (layer F.Cu) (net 6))
 (segment (start 134.62 62.948001) (end 135.89 61.678001) (width 0.25) (layer F.Cu) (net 6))
 (segment (start 134.62 66.04) (end 134.62 62.948001) (width 0.25) (layer F.Cu) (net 6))
 (segment (start 134.16999 60.858011) (end 135.89 59.138001) (width 0.25) (layer F.Cu) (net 7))
 (segment (start 134.16999 66.2264) (end 134.16999 60.858011) (width 0.25) (layer F.Cu) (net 7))
 (segment (start 134.437001 66.493411) (end 134.16999 66.2264) (width 0.25) (layer F.Cu) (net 7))
 (segment (start 134.437001 75.112999) (end 134.437001 66.493411) (width 0.25) (layer F.Cu) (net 7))
 (segment (start 133.35 76.2) (end 134.437001 75.112999) (width 0.25) (layer F.Cu) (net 7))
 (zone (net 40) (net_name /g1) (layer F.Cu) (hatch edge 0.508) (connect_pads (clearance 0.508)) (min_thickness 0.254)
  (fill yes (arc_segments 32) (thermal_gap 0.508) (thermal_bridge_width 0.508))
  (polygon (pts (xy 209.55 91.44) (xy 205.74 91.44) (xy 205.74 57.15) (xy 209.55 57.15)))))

